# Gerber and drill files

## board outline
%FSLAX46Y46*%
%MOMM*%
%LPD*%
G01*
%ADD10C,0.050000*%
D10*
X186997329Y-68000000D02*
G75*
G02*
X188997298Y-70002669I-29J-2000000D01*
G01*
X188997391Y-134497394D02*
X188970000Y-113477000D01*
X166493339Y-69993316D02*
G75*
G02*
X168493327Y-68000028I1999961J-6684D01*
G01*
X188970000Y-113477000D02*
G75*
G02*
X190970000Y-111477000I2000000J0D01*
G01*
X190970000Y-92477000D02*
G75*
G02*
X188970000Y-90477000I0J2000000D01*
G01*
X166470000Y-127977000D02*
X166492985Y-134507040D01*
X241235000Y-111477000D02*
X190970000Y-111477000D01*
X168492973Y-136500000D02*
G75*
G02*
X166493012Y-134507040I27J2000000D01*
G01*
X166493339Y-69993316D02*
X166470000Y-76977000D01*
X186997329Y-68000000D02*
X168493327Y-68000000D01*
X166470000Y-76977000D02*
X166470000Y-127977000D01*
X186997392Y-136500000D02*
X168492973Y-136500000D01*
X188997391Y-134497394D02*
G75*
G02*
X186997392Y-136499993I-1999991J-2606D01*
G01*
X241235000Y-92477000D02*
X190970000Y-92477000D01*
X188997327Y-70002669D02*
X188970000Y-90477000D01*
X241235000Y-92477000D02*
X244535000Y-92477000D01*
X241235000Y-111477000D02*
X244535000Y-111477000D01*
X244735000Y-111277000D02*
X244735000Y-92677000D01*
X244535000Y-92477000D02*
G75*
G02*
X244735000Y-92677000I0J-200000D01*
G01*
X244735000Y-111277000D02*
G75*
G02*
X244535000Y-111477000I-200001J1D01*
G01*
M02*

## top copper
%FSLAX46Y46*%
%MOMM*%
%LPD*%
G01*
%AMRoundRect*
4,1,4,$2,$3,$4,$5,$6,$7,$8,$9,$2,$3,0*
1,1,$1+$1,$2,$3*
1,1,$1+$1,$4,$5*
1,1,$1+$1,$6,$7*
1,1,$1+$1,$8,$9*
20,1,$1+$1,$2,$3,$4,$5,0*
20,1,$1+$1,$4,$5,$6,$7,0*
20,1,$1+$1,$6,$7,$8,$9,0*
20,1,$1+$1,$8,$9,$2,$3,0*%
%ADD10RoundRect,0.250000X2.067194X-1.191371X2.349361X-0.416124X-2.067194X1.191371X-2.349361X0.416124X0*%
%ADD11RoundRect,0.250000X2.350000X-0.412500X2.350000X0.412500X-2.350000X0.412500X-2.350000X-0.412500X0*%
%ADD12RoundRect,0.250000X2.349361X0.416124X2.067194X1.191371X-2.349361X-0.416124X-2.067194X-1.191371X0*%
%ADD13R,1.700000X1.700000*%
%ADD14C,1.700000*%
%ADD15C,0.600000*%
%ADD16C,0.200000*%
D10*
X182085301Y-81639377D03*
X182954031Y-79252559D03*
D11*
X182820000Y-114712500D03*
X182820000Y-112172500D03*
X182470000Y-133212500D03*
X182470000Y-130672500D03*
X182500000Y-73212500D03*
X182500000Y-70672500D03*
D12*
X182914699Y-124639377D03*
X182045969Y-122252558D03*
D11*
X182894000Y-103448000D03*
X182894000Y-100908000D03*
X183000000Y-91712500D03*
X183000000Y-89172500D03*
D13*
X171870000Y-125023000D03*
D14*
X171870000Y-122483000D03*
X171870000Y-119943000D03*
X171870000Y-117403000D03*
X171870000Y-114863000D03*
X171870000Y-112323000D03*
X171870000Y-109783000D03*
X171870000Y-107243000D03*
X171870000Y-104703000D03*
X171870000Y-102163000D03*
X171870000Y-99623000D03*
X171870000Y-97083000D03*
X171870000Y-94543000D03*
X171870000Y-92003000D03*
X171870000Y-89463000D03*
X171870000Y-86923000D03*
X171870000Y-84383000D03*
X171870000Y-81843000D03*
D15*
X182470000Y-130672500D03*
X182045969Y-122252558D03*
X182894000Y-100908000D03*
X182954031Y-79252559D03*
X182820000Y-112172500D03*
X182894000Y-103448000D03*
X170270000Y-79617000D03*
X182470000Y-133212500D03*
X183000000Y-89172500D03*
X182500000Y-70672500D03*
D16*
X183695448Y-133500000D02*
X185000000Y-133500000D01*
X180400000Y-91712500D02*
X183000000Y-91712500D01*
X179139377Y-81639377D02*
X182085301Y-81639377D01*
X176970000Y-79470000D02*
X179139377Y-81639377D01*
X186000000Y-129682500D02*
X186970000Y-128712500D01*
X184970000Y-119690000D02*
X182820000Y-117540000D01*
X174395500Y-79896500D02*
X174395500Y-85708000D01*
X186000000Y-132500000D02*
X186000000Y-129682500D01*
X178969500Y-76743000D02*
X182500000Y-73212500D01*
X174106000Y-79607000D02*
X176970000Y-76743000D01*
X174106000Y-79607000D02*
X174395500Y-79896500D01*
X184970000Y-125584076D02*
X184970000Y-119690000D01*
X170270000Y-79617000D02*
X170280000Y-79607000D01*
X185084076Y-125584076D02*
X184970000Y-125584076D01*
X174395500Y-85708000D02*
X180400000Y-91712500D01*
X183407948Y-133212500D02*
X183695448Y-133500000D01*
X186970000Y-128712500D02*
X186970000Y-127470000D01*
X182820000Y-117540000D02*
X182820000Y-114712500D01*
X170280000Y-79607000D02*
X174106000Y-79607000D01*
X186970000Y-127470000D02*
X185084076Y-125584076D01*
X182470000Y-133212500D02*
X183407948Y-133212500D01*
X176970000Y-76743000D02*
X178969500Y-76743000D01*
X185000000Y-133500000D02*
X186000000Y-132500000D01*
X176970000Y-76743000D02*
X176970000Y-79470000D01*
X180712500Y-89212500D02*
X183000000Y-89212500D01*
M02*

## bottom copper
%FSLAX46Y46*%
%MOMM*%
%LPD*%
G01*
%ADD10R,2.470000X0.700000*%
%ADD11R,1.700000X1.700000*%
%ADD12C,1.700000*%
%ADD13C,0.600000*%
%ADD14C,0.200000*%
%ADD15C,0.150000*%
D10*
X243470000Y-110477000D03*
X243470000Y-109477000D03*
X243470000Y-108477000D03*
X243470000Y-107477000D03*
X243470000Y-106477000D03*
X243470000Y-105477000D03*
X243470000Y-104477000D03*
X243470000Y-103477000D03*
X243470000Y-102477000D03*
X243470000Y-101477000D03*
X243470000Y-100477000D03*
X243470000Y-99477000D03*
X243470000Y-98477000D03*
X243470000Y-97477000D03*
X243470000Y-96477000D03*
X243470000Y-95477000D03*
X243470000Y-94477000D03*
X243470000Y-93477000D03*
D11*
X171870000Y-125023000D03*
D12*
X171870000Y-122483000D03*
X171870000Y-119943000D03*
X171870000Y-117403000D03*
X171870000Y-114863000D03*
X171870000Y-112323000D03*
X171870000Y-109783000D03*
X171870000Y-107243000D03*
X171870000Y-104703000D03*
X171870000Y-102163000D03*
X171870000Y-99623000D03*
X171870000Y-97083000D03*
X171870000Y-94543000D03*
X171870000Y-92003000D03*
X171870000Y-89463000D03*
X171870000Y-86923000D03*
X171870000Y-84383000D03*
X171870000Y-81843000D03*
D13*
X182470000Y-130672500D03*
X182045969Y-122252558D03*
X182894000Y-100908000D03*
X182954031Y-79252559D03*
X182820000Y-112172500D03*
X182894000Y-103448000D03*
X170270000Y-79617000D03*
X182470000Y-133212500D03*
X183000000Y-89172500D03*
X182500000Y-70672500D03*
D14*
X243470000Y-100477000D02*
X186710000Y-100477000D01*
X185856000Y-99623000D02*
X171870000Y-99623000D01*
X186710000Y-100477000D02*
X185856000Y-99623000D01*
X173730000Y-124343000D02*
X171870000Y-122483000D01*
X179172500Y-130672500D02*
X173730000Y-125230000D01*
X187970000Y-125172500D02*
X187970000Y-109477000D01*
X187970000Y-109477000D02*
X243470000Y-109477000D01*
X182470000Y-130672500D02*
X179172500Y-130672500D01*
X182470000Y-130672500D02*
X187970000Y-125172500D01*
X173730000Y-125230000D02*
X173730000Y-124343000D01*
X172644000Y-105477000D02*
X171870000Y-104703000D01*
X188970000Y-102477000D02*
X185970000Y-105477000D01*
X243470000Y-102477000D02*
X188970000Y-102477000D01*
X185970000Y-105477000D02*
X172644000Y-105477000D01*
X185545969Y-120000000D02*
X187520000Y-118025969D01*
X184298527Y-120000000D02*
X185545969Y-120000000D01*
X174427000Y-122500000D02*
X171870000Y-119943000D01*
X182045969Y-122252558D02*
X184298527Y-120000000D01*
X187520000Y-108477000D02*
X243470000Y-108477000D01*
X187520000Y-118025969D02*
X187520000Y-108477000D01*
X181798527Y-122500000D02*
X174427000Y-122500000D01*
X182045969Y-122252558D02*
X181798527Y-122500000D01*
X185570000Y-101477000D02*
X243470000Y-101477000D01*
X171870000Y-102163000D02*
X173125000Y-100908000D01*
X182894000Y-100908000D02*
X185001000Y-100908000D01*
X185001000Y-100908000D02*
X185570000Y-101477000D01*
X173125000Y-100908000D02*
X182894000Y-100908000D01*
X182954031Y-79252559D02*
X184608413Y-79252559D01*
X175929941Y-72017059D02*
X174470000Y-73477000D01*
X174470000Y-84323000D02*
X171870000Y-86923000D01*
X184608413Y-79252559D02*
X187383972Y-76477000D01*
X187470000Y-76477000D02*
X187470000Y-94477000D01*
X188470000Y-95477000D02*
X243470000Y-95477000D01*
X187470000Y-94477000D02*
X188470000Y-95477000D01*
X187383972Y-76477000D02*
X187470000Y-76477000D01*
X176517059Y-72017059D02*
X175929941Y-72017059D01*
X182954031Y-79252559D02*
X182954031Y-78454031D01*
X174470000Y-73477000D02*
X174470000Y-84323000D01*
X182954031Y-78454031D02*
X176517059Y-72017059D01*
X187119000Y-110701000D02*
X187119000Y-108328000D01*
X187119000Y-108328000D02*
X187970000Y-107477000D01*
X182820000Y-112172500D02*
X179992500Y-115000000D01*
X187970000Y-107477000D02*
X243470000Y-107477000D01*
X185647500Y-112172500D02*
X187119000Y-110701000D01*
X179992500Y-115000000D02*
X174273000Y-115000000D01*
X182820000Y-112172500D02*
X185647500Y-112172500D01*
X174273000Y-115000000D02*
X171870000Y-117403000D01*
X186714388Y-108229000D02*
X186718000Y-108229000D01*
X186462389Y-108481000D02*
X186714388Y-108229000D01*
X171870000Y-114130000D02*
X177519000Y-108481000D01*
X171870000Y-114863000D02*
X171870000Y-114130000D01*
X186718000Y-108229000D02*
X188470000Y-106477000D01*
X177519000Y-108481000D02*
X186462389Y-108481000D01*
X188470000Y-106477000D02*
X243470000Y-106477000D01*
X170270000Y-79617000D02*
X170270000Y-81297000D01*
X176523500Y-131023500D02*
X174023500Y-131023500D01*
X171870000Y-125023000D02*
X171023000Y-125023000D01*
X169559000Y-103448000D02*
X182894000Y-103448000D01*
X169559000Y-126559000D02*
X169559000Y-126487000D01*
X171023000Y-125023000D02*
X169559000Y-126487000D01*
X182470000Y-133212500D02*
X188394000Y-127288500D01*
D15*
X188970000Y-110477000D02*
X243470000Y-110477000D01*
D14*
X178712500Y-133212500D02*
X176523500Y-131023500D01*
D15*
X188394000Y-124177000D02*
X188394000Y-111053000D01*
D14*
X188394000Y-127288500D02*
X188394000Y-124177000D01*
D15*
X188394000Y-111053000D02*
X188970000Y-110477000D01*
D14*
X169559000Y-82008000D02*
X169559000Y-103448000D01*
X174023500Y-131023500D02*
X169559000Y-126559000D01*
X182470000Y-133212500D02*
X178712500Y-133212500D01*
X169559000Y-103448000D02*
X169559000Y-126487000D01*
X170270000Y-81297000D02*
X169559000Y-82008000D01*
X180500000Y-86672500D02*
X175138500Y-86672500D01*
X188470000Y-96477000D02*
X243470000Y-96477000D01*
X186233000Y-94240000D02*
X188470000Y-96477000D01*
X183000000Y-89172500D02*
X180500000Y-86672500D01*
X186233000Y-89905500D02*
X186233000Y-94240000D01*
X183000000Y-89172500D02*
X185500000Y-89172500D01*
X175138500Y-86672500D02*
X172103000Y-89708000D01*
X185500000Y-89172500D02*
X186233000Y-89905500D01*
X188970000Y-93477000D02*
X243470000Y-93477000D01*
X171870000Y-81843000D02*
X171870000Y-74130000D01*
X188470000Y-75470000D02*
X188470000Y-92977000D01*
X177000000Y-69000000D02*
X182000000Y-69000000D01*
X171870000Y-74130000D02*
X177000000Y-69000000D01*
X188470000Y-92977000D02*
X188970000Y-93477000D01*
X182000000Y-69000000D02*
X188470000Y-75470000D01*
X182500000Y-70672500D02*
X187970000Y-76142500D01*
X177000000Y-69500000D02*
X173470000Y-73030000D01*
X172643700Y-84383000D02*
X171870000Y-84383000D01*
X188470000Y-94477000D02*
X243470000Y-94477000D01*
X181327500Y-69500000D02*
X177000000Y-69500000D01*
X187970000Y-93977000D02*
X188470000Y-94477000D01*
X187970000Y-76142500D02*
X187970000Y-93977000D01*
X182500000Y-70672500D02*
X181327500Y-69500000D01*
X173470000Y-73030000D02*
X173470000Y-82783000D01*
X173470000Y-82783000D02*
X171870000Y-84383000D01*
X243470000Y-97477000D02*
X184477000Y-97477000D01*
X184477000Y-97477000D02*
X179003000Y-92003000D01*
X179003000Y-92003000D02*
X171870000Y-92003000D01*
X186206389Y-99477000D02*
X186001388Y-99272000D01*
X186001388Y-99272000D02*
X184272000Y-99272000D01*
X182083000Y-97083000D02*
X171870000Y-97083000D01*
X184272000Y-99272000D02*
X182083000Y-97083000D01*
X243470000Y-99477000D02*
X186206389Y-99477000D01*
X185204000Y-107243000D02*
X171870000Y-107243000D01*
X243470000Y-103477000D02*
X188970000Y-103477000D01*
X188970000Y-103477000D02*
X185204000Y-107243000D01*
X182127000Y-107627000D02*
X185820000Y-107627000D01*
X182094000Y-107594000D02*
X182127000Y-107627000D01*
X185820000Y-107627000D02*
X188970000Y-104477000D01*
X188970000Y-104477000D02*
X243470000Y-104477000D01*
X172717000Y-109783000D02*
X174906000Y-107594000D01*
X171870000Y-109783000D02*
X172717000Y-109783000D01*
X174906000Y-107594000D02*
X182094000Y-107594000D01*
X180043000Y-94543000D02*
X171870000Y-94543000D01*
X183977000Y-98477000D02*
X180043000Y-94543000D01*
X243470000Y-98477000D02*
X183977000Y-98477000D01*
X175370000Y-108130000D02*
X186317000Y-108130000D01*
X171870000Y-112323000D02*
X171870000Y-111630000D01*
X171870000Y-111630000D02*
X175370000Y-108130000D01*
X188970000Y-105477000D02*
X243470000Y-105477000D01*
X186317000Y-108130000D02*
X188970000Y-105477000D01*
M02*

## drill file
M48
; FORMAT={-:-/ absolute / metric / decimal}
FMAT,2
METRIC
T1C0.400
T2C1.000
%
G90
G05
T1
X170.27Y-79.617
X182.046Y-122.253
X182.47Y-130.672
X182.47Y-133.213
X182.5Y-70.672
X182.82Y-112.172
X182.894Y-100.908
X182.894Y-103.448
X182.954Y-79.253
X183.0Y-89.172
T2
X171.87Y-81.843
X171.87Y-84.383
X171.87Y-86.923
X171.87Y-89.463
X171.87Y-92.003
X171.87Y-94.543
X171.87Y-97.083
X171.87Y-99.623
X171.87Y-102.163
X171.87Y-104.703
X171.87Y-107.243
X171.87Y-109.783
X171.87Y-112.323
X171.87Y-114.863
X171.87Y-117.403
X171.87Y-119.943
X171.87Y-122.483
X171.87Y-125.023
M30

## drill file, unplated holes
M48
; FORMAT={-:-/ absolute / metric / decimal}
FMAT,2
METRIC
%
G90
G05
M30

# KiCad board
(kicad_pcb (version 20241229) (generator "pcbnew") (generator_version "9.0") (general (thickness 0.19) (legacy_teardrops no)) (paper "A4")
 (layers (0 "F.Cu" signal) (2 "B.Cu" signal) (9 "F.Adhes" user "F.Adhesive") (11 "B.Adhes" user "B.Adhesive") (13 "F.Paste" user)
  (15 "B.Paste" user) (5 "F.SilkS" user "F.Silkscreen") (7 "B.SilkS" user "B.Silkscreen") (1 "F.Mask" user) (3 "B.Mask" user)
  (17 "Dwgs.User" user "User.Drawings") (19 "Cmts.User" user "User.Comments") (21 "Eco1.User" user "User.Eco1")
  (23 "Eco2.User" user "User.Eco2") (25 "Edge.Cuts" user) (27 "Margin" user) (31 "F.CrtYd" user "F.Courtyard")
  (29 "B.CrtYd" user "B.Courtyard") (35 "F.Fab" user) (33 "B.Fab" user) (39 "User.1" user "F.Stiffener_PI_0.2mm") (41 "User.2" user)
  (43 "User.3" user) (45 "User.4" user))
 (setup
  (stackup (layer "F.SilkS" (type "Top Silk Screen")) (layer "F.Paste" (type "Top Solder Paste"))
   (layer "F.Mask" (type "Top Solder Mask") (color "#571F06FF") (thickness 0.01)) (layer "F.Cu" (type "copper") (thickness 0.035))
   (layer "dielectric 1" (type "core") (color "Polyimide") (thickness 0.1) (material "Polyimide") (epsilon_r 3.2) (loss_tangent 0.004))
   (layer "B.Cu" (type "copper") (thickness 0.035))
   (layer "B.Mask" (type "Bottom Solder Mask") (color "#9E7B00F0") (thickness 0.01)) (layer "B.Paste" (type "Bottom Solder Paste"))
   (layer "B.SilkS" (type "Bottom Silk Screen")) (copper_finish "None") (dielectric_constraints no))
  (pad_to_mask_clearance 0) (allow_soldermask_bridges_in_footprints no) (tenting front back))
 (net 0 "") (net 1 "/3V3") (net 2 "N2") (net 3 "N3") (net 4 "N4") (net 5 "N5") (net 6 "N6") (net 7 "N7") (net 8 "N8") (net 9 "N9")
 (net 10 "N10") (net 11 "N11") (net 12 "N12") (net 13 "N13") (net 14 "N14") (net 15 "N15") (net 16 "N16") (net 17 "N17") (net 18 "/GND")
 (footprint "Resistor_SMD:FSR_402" (layer "F.Cu") (at 182.5 80.5 70)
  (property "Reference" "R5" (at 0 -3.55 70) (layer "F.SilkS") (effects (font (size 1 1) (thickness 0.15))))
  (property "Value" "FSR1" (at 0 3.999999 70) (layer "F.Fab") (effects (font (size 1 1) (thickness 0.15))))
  (pad "1" smd roundrect (at -1.2125 0 70) (size 1.325 5.2) (layers "F.Cu" "F.Mask" "F.Paste") (roundrect_rratio 0.188679) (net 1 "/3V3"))
  (pad "2" smd roundrect (at 1.327499 0 70) (size 1.325 5.2) (layers "F.Cu" "F.Mask" "F.Paste") (roundrect_rratio 0.188679) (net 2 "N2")))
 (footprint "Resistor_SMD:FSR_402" (layer "F.Cu") (at 182.82 113.5 90)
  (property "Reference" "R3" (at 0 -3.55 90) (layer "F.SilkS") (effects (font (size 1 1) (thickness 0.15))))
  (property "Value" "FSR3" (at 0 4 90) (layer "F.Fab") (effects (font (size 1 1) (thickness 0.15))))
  (pad "1" smd roundrect (at -1.2125 0 90) (size 1.325 5.2) (layers "F.Cu" "F.Mask" "F.Paste") (roundrect_rratio 0.188679) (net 1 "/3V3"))
  (pad "2" smd roundrect (at 1.3275 0 90) (size 1.325 5.2) (layers "F.Cu" "F.Mask" "F.Paste") (roundrect_rratio 0.188679) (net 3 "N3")))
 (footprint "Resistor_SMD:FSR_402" (layer "F.Cu") (at 182.47 132 90)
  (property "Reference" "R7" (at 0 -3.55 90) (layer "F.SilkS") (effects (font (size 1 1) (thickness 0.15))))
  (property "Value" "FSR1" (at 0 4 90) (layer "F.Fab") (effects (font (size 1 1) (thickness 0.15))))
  (pad "1" smd roundrect (at -1.2125 0 90) (size 1.325 5.2) (layers "F.Cu" "F.Mask" "F.Paste") (roundrect_rratio 0.188679) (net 1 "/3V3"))
  (pad "2" smd roundrect (at 1.3275 0 90) (size 1.325 5.2) (layers "F.Cu" "F.Mask" "F.Paste") (roundrect_rratio 0.188679) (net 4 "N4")))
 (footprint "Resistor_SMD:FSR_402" (layer "F.Cu") (at 182.5 72 90)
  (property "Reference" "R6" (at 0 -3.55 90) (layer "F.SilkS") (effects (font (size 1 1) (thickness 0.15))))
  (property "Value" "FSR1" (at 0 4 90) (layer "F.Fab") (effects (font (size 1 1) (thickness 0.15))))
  (pad "1" smd roundrect (at -1.2125 0 90) (size 1.325 5.2) (layers "F.Cu" "F.Mask" "F.Paste") (roundrect_rratio 0.188679) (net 1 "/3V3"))
  (pad "2" smd roundrect (at 1.3275 0 90) (size 1.325 5.2) (layers "F.Cu" "F.Mask" "F.Paste") (roundrect_rratio 0.188679) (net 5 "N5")))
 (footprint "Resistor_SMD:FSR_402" (layer "F.Cu") (at 182.5 123.5 110)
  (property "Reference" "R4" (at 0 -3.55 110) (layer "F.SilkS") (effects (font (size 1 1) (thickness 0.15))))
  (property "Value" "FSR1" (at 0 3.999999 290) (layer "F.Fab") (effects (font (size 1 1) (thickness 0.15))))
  (pad "1" smd roundrect (at -1.2125 0 110) (size 1.325 5.2) (layers "F.Cu" "F.Mask" "F.Paste") (roundrect_rratio 0.188679) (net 1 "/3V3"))
  (pad "2" smd roundrect (at 1.3275 0.000001 110) (size 1.325 5.2) (layers "F.Cu" "F.Mask" "F.Paste") (roundrect_rratio 0.188679)
   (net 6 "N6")))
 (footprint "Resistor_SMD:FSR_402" (layer "F.Cu") (at 182.894 102.2355 90)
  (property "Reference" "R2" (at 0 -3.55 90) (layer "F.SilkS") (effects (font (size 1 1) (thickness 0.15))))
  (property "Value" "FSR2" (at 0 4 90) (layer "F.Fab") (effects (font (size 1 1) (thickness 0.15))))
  (pad "1" smd roundrect (at -1.2125 0 90) (size 1.325 5.2) (layers "F.Cu" "F.Mask" "F.Paste") (roundrect_rratio 0.188679) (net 1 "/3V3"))
  (pad "2" smd roundrect (at 1.3275 0 90) (size 1.325 5.2) (layers "F.Cu" "F.Mask" "F.Paste") (roundrect_rratio 0.188679) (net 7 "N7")))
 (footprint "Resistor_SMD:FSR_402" (layer "F.Cu") (at 183 90.5 90)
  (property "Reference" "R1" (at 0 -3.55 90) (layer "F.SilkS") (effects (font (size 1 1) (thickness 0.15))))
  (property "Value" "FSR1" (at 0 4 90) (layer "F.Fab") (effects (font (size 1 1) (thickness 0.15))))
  (pad "1" smd roundrect (at -1.2125 0 90) (size 1.325 5.2) (layers "F.Cu" "F.Mask" "F.Paste") (roundrect_rratio 0.188679) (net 1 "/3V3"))
  (pad "2" smd roundrect (at 1.3275 0 90) (size 1.325 5.2) (layers "F.Cu" "F.Mask" "F.Paste") (roundrect_rratio 0.188679) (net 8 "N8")))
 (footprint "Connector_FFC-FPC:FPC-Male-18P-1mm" (layer "B.Cu") (at 243.43 102.387 90)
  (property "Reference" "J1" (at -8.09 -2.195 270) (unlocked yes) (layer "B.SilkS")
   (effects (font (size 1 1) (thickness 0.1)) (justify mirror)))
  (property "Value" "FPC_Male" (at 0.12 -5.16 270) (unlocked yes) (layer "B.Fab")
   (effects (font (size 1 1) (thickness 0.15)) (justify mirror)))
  (fp_line (start 9.91 -2.195) (end 9.91 1.105) (stroke (width 0.05) (type default)) (layer "Edge.Cuts"))
  (fp_line (start -9.09 -2.195) (end -9.09 1.105) (stroke (width 0.05) (type default)) (layer "Edge.Cuts"))
  (fp_line (start -8.89 1.305) (end 9.71 1.305) (stroke (width 0.05) (type default)) (layer "Edge.Cuts"))
  (fp_arc (start 9.91 1.105) (mid 9.851421 1.246421) (end 9.71 1.305) (stroke (width 0.05) (type default)) (layer "Edge.Cuts"))
  (fp_arc (start -8.89 1.305) (mid -9.031421 1.246421) (end -9.09 1.105) (stroke (width 0.05) (type default)) (layer "Edge.Cuts"))
  (pad "1" smd rect (at -8.09 0.04) (size 2.47 0.7) (layers "B.Cu" "B.Mask" "B.Paste") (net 1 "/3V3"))
  (pad "2" smd rect (at -7.09 0.04) (size 2.47 0.7) (layers "B.Cu" "B.Mask" "B.Paste") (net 4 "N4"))
  (pad "3" smd rect (at -6.09 0.04) (size 2.47 0.7) (layers "B.Cu" "B.Mask" "B.Paste") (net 6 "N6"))
  (pad "4" smd rect (at -5.09 0.04) (size 2.47 0.7) (layers "B.Cu" "B.Mask" "B.Paste") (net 3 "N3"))
  (pad "5" smd rect (at -4.09 0.04) (size 2.47 0.7) (layers "B.Cu" "B.Mask" "B.Paste") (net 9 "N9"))
  (pad "6" smd rect (at -3.09 0.04) (size 2.47 0.7) (layers "B.Cu" "B.Mask" "B.Paste") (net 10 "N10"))
  (pad "7" smd rect (at -2.09 0.04) (size 2.47 0.7) (layers "B.Cu" "B.Mask" "B.Paste") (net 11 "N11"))
  (pad "8" smd rect (at -1.09 0.04) (size 2.47 0.7) (layers "B.Cu" "B.Mask" "B.Paste") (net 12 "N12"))
  (pad "9" smd rect (at -0.09 0.04) (size 2.47 0.7) (layers "B.Cu" "B.Mask" "B.Paste") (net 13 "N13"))
  (pad "10" smd rect (at 0.91 0.04) (size 2.47 0.7) (layers "B.Cu" "B.Mask" "B.Paste") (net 7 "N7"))
  (pad "11" smd rect (at 1.91 0.04) (size 2.47 0.7) (layers "B.Cu" "B.Mask" "B.Paste") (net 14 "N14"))
  (pad "12" smd rect (at 2.91 0.04) (size 2.47 0.7) (layers "B.Cu" "B.Mask" "B.Paste") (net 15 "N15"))
  (pad "13" smd rect (at 3.91 0.04) (size 2.47 0.7) (layers "B.Cu" "B.Mask" "B.Paste") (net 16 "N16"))
  (pad "14" smd rect (at 4.91 0.04) (size 2.47 0.7) (layers "B.Cu" "B.Mask" "B.Paste") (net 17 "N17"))
  (pad "15" smd rect (at 5.91 0.04) (size 2.47 0.7) (layers "B.Cu" "B.Mask" "B.Paste") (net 8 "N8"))
  (pad "16" smd rect (at 6.91 0.04) (size 2.47 0.7) (layers "B.Cu" "B.Mask" "B.Paste") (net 2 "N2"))
  (pad "17" smd rect (at 7.91 0.04) (size 2.47 0.7) (layers "B.Cu" "B.Mask" "B.Paste") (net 5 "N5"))
  (pad "18" smd rect (at 8.91 0.04) (size 2.47 0.7) (layers "B.Cu" "B.Mask" "B.Paste") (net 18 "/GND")))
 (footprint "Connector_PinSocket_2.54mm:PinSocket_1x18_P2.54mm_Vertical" (layer "B.Cu") (at 171.87 125.023)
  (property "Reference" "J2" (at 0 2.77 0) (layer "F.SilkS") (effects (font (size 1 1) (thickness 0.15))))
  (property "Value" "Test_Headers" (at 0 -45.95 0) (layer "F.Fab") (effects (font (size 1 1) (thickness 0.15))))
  (pad "1" thru_hole rect (at 0 0) (size 1.7 1.7) (drill 1) (layers "*.Cu" "*.Mask") (remove_unused_layers no) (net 1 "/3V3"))
  (pad "2" thru_hole circle (at 0 -2.54) (size 1.7 1.7) (drill 1) (layers "*.Cu" "*.Mask") (remove_unused_layers no) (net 4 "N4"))
  (pad "3" thru_hole circle (at 0 -5.08) (size 1.7 1.7) (drill 1) (layers "*.Cu" "*.Mask") (remove_unused_layers no) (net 6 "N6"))
  (pad "4" thru_hole circle (at 0 -7.62) (size 1.7 1.7) (drill 1) (layers "*.Cu" "*.Mask") (remove_unused_layers no) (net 3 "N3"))
  (pad "5" thru_hole circle (at 0 -10.16) (size 1.7 1.7) (drill 1) (layers "*.Cu" "*.Mask") (remove_unused_layers no) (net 9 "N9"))
  (pad "6" thru_hole circle (at 0 -12.7) (size 1.7 1.7) (drill 1) (layers "*.Cu" "*.Mask") (remove_unused_layers no) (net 10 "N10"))
  (pad "7" thru_hole circle (at 0 -15.24) (size 1.7 1.7) (drill 1) (layers "*.Cu" "*.Mask") (remove_unused_layers no) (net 11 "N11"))
  (pad "8" thru_hole circle (at 0 -17.78) (size 1.7 1.7) (drill 1) (layers "*.Cu" "*.Mask") (remove_unused_layers no) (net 12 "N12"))
  (pad "9" thru_hole circle (at 0 -20.32) (size 1.7 1.7) (drill 1) (layers "*.Cu" "*.Mask") (remove_unused_layers no) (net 13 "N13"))
  (pad "10" thru_hole circle (at 0 -22.86) (size 1.7 1.7) (drill 1) (layers "*.Cu" "*.Mask") (remove_unused_layers no) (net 7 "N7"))
  (pad "11" thru_hole circle (at 0 -25.4) (size 1.7 1.7) (drill 1) (layers "*.Cu" "*.Mask") (remove_unused_layers no) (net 14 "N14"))
  (pad "12" thru_hole circle (at 0 -27.94) (size 1.7 1.7) (drill 1) (layers "*.Cu" "*.Mask") (remove_unused_layers no) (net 15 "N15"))
  (pad "13" thru_hole circle (at 0 -30.48) (size 1.7 1.7) (drill 1) (layers "*.Cu" "*.Mask") (remove_unused_layers no) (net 16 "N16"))
  (pad "14" thru_hole circle (at 0 -33.02) (size 1.7 1.7) (drill 1) (layers "*.Cu" "*.Mask") (remove_unused_layers no) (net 17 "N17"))
  (pad "15" thru_hole circle (at 0 -35.56) (size 1.7 1.7) (drill 1) (layers "*.Cu" "*.Mask") (remove_unused_layers no) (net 8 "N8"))
  (pad "16" thru_hole circle (at 0 -38.1) (size 1.7 1.7) (drill 1) (layers "*.Cu" "*.Mask") (remove_unused_layers no) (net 2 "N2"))
  (pad "17" thru_hole circle (at 0 -40.64) (size 1.7 1.7) (drill 1) (layers "*.Cu" "*.Mask") (remove_unused_layers no) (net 5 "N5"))
  (pad "18" thru_hole circle (at 0 -43.18) (size 1.7 1.7) (drill 1) (layers "*.Cu" "*.Mask") (remove_unused_layers no) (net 18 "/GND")))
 (gr_arc (start 186.997329 68) (mid 188.412486 68.58673) (end 188.997327 70.002669) (stroke (width 0.05) (type default)) (layer "Edge.Cuts"))
 (gr_line (start 188.997391 134.497394) (end 188.97 113.477) (stroke (width 0.05) (type default)) (layer "Edge.Cuts"))
 (gr_arc (start 166.493339 69.993316) (mid 167.081479 68.583426) (end 168.493327 68) (stroke (width 0.05) (type default))
  (layer "Edge.Cuts"))
 (gr_arc (start 188.97 113.477) (mid 189.555786 112.062786) (end 190.97 111.477) (stroke (width 0.05) (type default)) (layer "Edge.Cuts"))
 (gr_arc (start 190.97 92.477) (mid 189.555786 91.891214) (end 188.97 90.477) (stroke (width 0.05) (type default)) (layer "Edge.Cuts"))
 (gr_line (start 166.47 127.977) (end 166.492985 134.50704) (stroke (width 0.05) (type default)) (layer "Edge.Cuts"))
 (gr_line (start 241.235 111.477) (end 190.97 111.477) (stroke (width 0.05) (type default)) (layer "Edge.Cuts"))
 (gr_arc (start 168.492973 136.5) (mid 167.081268 135.916691) (end 166.492985 134.50704) (stroke (width 0.05) (type default))
  (layer "Edge.Cuts"))
 (gr_line (start 166.493339 69.993316) (end 166.47 76.977) (stroke (width 0.05) (type default)) (layer "Edge.Cuts"))
 (gr_line (start 186.997329 68) (end 168.493327 68) (stroke (width 0.05) (type default)) (layer "Edge.Cuts"))
 (gr_line (start 166.47 76.977) (end 166.47 127.977) (stroke (width 0.05) (type default)) (layer "Edge.Cuts"))
 (gr_line (start 186.997392 136.5) (end 168.492973 136.5) (stroke (width 0.05) (type default)) (layer "Edge.Cuts"))
 (gr_arc (start 188.997391 134.497394) (mid 188.412527 135.913292) (end 186.997392 136.5) (stroke (width 0.05) (type default))
  (layer "Edge.Cuts"))
 (gr_line (start 241.235 92.477) (end 190.97 92.477) (stroke (width 0.05) (type default)) (layer "Edge.Cuts"))
 (gr_line (start 188.997327 70.002669) (end 188.97 90.477) (stroke (width 0.05) (type default)) (layer "Edge.Cuts"))
 (segment (start 243.47 100.477) (end 186.71 100.477) (width 0.2) (layer "B.Cu") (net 14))
 (segment (start 185.856 99.623) (end 171.87 99.623) (width 0.2) (layer "B.Cu") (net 14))
 (segment (start 186.71 100.477) (end 185.856 99.623) (width 0.2) (layer "B.Cu") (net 14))
 (via (at 182.47 130.6725) (size 0.6) (drill 0.4) (layers "F.Cu" "B.Cu") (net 4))
 (segment (start 173.73 124.343) (end 171.87 122.483) (width 0.2) (layer "B.Cu") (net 4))
 (segment (start 179.1725 130.6725) (end 173.73 125.23) (width 0.2) (layer "B.Cu") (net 4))
 (segment (start 187.97 125.1725) (end 187.97 109.477) (width 0.2) (layer "B.Cu") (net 4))
 (segment (start 187.97 109.477) (end 243.47 109.477) (width 0.2) (layer "B.Cu") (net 4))
 (segment (start 182.47 130.6725) (end 179.1725 130.6725) (width 0.2) (layer "B.Cu") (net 4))
 (segment (start 182.47 130.6725) (end 187.97 125.1725) (width 0.2) (layer "B.Cu") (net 4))
 (segment (start 173.73 125.23) (end 173.73 124.343) (width 0.2) (layer "B.Cu") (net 4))
 (segment (start 172.644 105.477) (end 171.87 104.703) (width 0.2) (layer "B.Cu") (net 13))
 (segment (start 188.97 102.477) (end 185.97 105.477) (width 0.2) (layer "B.Cu") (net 13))
 (segment (start 243.47 102.477) (end 188.97 102.477) (width 0.2) (layer "B.Cu") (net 13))
 (segment (start 185.97 105.477) (end 172.644 105.477) (width 0.2) (layer "B.Cu") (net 13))
 (via (at 182.045969 122.252558) (size 0.6) (drill 0.4) (layers "F.Cu" "B.Cu") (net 6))
 (segment (start 185.545969 120) (end 187.52 118.025969) (width 0.2) (layer "B.Cu") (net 6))
 (segment (start 184.298527 120) (end 185.545969 120) (width 0.2) (layer "B.Cu") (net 6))
 (segment (start 174.427 122.5) (end 171.87 119.943) (width 0.2) (layer "B.Cu") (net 6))
 (segment (start 182.045969 122.252558) (end 184.298527 120) (width 0.2) (layer "B.Cu") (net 6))
 (segment (start 187.52 108.477) (end 243.47 108.477) (width 0.2) (layer "B.Cu") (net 6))
 (segment (start 187.52 118.025969) (end 187.52 108.477) (width 0.2) (layer "B.Cu") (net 6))
 (segment (start 181.798527 122.5) (end 174.427 122.5) (width 0.2) (layer "B.Cu") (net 6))
 (segment (start 182.045969 122.252558) (end 181.798527 122.5) (width 0.2) (layer "B.Cu") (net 6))
 (via (at 182.894 100.908) (size 0.6) (drill 0.4) (layers "F.Cu" "B.Cu") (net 7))
 (segment (start 185.57 101.477) (end 243.47 101.477) (width 0.2) (layer "B.Cu") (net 7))
 (segment (start 171.87 102.163) (end 173.125 100.908) (width 0.2) (layer "B.Cu") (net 7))
 (segment (start 182.894 100.908) (end 185.001 100.908) (width 0.2) (layer "B.Cu") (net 7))
 (segment (start 185.001 100.908) (end 185.57 101.477) (width 0.2) (layer "B.Cu") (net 7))
 (segment (start 173.125 100.908) (end 182.894 100.908) (width 0.2) (layer "B.Cu") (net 7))
 (via (at 182.954031 79.252559) (size 0.6) (drill 0.4) (layers "F.Cu" "B.Cu") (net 2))
 (segment (start 182.954031 79.252559) (end 184.608413 79.252559) (width 0.2) (layer "B.Cu") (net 2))
 (segment (start 175.929941 72.017059) (end 174.47 73.477) (width 0.2) (layer "B.Cu") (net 2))
 (segment (start 174.47 84.323) (end 171.87 86.923) (width 0.2) (layer "B.Cu") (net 2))
 (segment (start 184.608413 79.252559) (end 187.383972 76.477) (width 0.2) (layer "B.Cu") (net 2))
 (segment (start 187.47 76.477) (end 187.47 94.477) (width 0.2) (layer "B.Cu") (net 2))
 (segment (start 188.47 95.477) (end 243.47 95.477) (width 0.2) (layer "B.Cu") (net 2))
 (segment (start 187.47 94.477) (end 188.47 95.477) (width 0.2) (layer "B.Cu") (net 2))
 (segment (start 187.383972 76.477) (end 187.47 76.477) (width 0.2) (layer "B.Cu") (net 2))
 (segment (start 176.517059 72.017059) (end 175.929941 72.017059) (width 0.2) (layer "B.Cu") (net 2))
 (segment (start 182.954031 79.252559) (end 182.954031 78.454031) (width 0.2) (layer "B.Cu") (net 2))
 (segment (start 174.47 73.477) (end 174.47 84.323) (width 0.2) (layer "B.Cu") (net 2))
 (segment (start 182.954031 78.454031) (end 176.517059 72.017059) (width 0.2) (layer "B.Cu") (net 2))
 (via (at 182.82 112.1725) (size 0.6) (drill 0.4) (layers "F.Cu" "B.Cu") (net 3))
 (segment (start 187.119 110.701) (end 187.119 108.328) (width 0.2) (layer "B.Cu") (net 3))
 (segment (start 187.119 108.328) (end 187.97 107.477) (width 0.2) (layer "B.Cu") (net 3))
 (segment (start 182.82 112.1725) (end 179.9925 115) (width 0.2) (layer "B.Cu") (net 3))
 (segment (start 187.97 107.477) (end 243.47 107.477) (width 0.2) (layer "B.Cu") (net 3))
 (segment (start 185.6475 112.1725) (end 187.119 110.701) (width 0.2) (layer "B.Cu") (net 3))
 (segment (start 179.9925 115) (end 174.273 115) (width 0.2) (layer "B.Cu") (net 3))
 (segment (start 182.82 112.1725) (end 185.6475 112.1725) (width 0.2) (layer "B.Cu") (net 3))
 (segment (start 174.273 115) (end 171.87 117.403) (width 0.2) (layer "B.Cu") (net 3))
 (segment (start 186.714388 108.229) (end 186.718 108.229) (width 0.2) (layer "B.Cu") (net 9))
 (segment (start 186.462389 108.481) (end 186.714388 108.229) (width 0.2) (layer "B.Cu") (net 9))
 (segment (start 171.87 114.13) (end 177.519 108.481) (width 0.2) (layer "B.Cu") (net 9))
 (segment (start 171.87 114.863) (end 171.87 114.13) (width 0.2) (layer "B.Cu") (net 9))
 (segment (start 186.718 108.229) (end 188.47 106.477) (width 0.2) (layer "B.Cu") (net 9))
 (segment (start 177.519 108.481) (end 186.462389 108.481) (width 0.2) (layer "B.Cu") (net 9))
 (segment (start 188.47 106.477) (end 243.47 106.477) (width 0.2) (layer "B.Cu") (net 9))
 (segment (start 183.695448 133.5) (end 185 133.5) (width 0.2) (layer "F.Cu") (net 1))
 (segment (start 180.4 91.7125) (end 183 91.7125) (width 0.2) (layer "F.Cu") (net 1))
 (segment (start 179.139377 81.639377) (end 182.085301 81.639377) (width 0.2) (layer "F.Cu") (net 1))
 (segment (start 176.97 79.47) (end 179.139377 81.639377) (width 0.2) (layer "F.Cu") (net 1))
 (segment (start 186 129.6825) (end 186.97 128.7125) (width 0.2) (layer "F.Cu") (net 1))
 (segment (start 184.97 119.69) (end 182.82 117.54) (width 0.2) (layer "F.Cu") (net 1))
 (segment (start 174.3955 79.8965) (end 174.3955 85.708) (width 0.2) (layer "F.Cu") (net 1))
 (segment (start 186 132.5) (end 186 129.6825) (width 0.2) (layer "F.Cu") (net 1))
 (segment (start 178.9695 76.743) (end 182.5 73.2125) (width 0.2) (layer "F.Cu") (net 1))
 (segment (start 174.106 79.607) (end 176.97 76.743) (width 0.2) (layer "F.Cu") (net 1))
 (segment (start 174.106 79.607) (end 174.3955 79.8965) (width 0.2) (layer "F.Cu") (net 1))
 (segment (start 184.97 125.584076) (end 184.97 119.69) (width 0.2) (layer "F.Cu") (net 1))
 (segment (start 170.27 79.617) (end 170.28 79.607) (width 0.2) (layer "F.Cu") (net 1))
 (segment (start 185.084076 125.584076) (end 184.97 125.584076) (width 0.2) (layer "F.Cu") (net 1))
 (segment (start 174.3955 85.708) (end 180.4 91.7125) (width 0.2) (layer "F.Cu") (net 1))
 (segment (start 183.407948 133.2125) (end 183.695448 133.5) (width 0.2) (layer "F.Cu") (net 1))
 (segment (start 186.97 128.7125) (end 186.97 127.47) (width 0.2) (layer "F.Cu") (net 1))
 (segment (start 182.82 117.54) (end 182.82 114.7125) (width 0.2) (layer "F.Cu") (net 1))
 (segment (start 170.28 79.607) (end 174.106 79.607) (width 0.2) (layer "F.Cu") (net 1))
 (segment (start 186.97 127.47) (end 185.084076 125.584076) (width 0.2) (layer "F.Cu") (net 1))
 (segment (start 182.47 133.2125) (end 183.407948 133.2125) (width 0.2) (layer "F.Cu") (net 1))
 (segment (start 176.97 76.743) (end 178.9695 76.743) (width 0.2) (layer "F.Cu") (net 1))
 (segment (start 185 133.5) (end 186 132.5) (width 0.2) (layer "F.Cu") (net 1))
 (segment (start 176.97 76.743) (end 176.97 79.47) (width 0.2) (layer "F.Cu") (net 1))
 (via (at 182.894 103.448) (size 0.6) (drill 0.4) (layers "F.Cu" "B.Cu") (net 1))
 (via (at 170.27 79.617) (size 0.6) (drill 0.4) (layers "F.Cu" "B.Cu") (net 1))
 (via (at 182.47 133.2125) (size 0.6) (drill 0.4) (layers "F.Cu" "B.Cu") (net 1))
 (segment (start 170.27 79.617) (end 170.27 81.297) (width 0.2) (layer "B.Cu") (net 1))
 (segment (start 176.5235 131.0235) (end 174.0235 131.0235) (width 0.2) (layer "B.Cu") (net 1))
 (segment (start 171.87 125.023) (end 171.023 125.023) (width 0.2) (layer "B.Cu") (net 1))
 (segment (start 169.559 103.448) (end 182.894 103.448) (width 0.2) (layer "B.Cu") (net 1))
 (segment (start 169.559 126.559) (end 169.559 126.487) (width 0.2) (layer "B.Cu") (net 1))
 (segment (start 171.023 125.023) (end 169.559 126.487) (width 0.2) (layer "B.Cu") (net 1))
 (segment (start 182.47 133.2125) (end 188.394 127.2885) (width 0.2) (layer "B.Cu") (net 1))
 (segment (start 188.97 110.477) (end 243.47 110.477) (width 0.15) (layer "B.Cu") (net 1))
 (segment (start 178.7125 133.2125) (end 176.5235 131.0235) (width 0.2) (layer "B.Cu") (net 1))
 (segment (start 188.394 124.177) (end 188.394 111.053) (width 0.15) (layer "B.Cu") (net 1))
 (segment (start 188.394 127.2885) (end 188.394 124.177) (width 0.2) (layer "B.Cu") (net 1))
 (segment (start 188.394 111.053) (end 188.97 110.477) (width 0.15) (layer "B.Cu") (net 1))
 (segment (start 169.559 82.008) (end 169.559 103.448) (width 0.2) (layer "B.Cu") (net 1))
 (segment (start 174.0235 131.0235) (end 169.559 126.559) (width 0.2) (layer "B.Cu") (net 1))
 (segment (start 182.47 133.2125) (end 178.7125 133.2125) (width 0.2) (layer "B.Cu") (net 1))
 (segment (start 169.559 103.448) (end 169.559 126.487) (width 0.2) (layer "B.Cu") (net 1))
 (segment (start 170.27 81.297) (end 169.559 82.008) (width 0.2) (layer "B.Cu") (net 1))
 (segment (start 180.7125 89.2125) (end 183 89.2125) (width 0.2) (layer "F.Cu") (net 8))
 (via (at 183 89.1725) (size 0.6) (drill 0.4) (layers "F.Cu" "B.Cu") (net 8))
 (segment (start 180.5 86.6725) (end 175.1385 86.6725) (width 0.2) (layer "B.Cu") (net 8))
 (segment (start 188.47 96.477) (end 243.47 96.477) (width 0.2) (layer "B.Cu") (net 8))
 (segment (start 186.233 94.24) (end 188.47 96.477) (width 0.2) (layer "B.Cu") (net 8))
 (segment (start 183 89.1725) (end 180.5 86.6725) (width 0.2) (layer "B.Cu") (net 8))
 (segment (start 186.233 89.9055) (end 186.233 94.24) (width 0.2) (layer "B.Cu") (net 8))
 (segment (start 183 89.1725) (end 185.5 89.1725) (width 0.2) (layer "B.Cu") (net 8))
 (segment (start 175.1385 86.6725) (end 172.103 89.708) (width 0.2) (layer "B.Cu") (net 8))
 (segment (start 185.5 89.1725) (end 186.233 89.9055) (width 0.2) (layer "B.Cu") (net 8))
 (segment (start 188.97 93.477) (end 243.47 93.477) (width 0.2) (layer "B.Cu") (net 18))
 (segment (start 171.87 81.843) (end 171.87 74.13) (width 0.2) (layer "B.Cu") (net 18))
 (segment (start 188.47 75.47) (end 188.47 92.977) (width 0.2) (layer "B.Cu") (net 18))
 (segment (start 177 69) (end 182 69) (width 0.2) (layer "B.Cu") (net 18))
 (segment (start 171.87 74.13) (end 177 69) (width 0.2) (layer "B.Cu") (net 18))
 (segment (start 188.47 92.977) (end 188.97 93.477) (width 0.2) (layer "B.Cu") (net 18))
 (segment (start 182 69) (end 188.47 75.47) (width 0.2) (layer "B.Cu") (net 18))
 (via (at 182.5 70.6725) (size 0.6) (drill 0.4) (layers "F.Cu" "B.Cu") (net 5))
 (segment (start 182.5 70.6725) (end 187.97 76.1425) (width 0.2) (layer "B.Cu") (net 5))
 (segment (start 177 69.5) (end 173.47 73.03) (width 0.2) (layer "B.Cu") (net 5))
 (segment (start 172.6437 84.383) (end 171.87 84.383) (width 0.2) (layer "B.Cu") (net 5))
 (segment (start 188.47 94.477) (end 243.47 94.477) (width 0.2) (layer "B.Cu") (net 5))
 (segment (start 181.3275 69.5) (end 177 69.5) (width 0.2) (layer "B.Cu") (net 5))
 (segment (start 187.97 93.977) (end 188.47 94.477) (width 0.2) (layer "B.Cu") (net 5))
 (segment (start 187.97 76.1425) (end 187.97 93.977) (width 0.2) (layer "B.Cu") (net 5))
 (segment (start 182.5 70.6725) (end 181.3275 69.5) (width 0.2) (layer "B.Cu") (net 5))
 (segment (start 173.47 73.03) (end 173.47 82.783) (width 0.2) (layer "B.Cu") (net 5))
 (segment (start 173.47 82.783) (end 171.87 84.383) (width 0.2) (layer "B.Cu") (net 5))
 (segment (start 243.47 97.477) (end 184.477 97.477) (width 0.2) (layer "B.Cu") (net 17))
 (segment (start 184.477 97.477) (end 179.003 92.003) (width 0.2) (layer "B.Cu") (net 17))
 (segment (start 179.003 92.003) (end 171.87 92.003) (width 0.2) (layer "B.Cu") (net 17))
 (segment (start 186.206389 99.477) (end 186.001388 99.272) (width 0.2) (layer "B.Cu") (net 15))
 (segment (start 186.001388 99.272) (end 184.272 99.272) (width 0.2) (layer "B.Cu") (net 15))
 (segment (start 182.083 97.083) (end 171.87 97.083) (width 0.2) (layer "B.Cu") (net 15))
 (segment (start 184.272 99.272) (end 182.083 97.083) (width 0.2) (layer "B.Cu") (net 15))
 (segment (start 243.47 99.477) (end 186.206389 99.477) (width 0.2) (layer "B.Cu") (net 15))
 (segment (start 185.204 107.243) (end 171.87 107.243) (width 0.2) (layer "B.Cu") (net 12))
 (segment (start 243.47 103.477) (end 188.97 103.477) (width 0.2) (layer "B.Cu") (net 12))
 (segment (start 188.97 103.477) (end 185.204 107.243) (width 0.2) (layer "B.Cu") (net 12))
 (segment (start 182.127 107.627) (end 185.82 107.627) (width 0.2) (layer "B.Cu") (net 11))
 (segment (start 182.094 107.594) (end 182.127 107.627) (width 0.2) (layer "B.Cu") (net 11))
 (segment (start 185.82 107.627) (end 188.97 104.477) (width 0.2) (layer "B.Cu") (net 11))
 (segment (start 188.97 104.477) (end 243.47 104.477) (width 0.2) (layer "B.Cu") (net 11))
 (segment (start 172.717 109.783) (end 174.906 107.594) (width 0.2) (layer "B.Cu") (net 11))
 (segment (start 171.87 109.783) (end 172.717 109.783) (width 0.2) (layer "B.Cu") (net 11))
 (segment (start 174.906 107.594) (end 182.094 107.594) (width 0.2) (layer "B.Cu") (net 11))
 (segment (start 180.043 94.543) (end 171.87 94.543) (width 0.2) (layer "B.Cu") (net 16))
 (segment (start 183.977 98.477) (end 180.043 94.543) (width 0.2) (layer "B.Cu") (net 16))
 (segment (start 243.47 98.477) (end 183.977 98.477) (width 0.2) (layer "B.Cu") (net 16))
 (segment (start 175.37 108.13) (end 186.317 108.13) (width 0.2) (layer "B.Cu") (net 10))
 (segment (start 171.87 112.323) (end 171.87 111.63) (width 0.2) (layer "B.Cu") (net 10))
 (segment (start 171.87 111.63) (end 175.37 108.13) (width 0.2) (layer "B.Cu") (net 10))
 (segment (start 188.97 105.477) (end 243.47 105.477) (width 0.2) (layer "B.Cu") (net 10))
 (segment (start 186.317 108.13) (end 188.97 105.477) (width 0.2) (layer "B.Cu") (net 10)))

